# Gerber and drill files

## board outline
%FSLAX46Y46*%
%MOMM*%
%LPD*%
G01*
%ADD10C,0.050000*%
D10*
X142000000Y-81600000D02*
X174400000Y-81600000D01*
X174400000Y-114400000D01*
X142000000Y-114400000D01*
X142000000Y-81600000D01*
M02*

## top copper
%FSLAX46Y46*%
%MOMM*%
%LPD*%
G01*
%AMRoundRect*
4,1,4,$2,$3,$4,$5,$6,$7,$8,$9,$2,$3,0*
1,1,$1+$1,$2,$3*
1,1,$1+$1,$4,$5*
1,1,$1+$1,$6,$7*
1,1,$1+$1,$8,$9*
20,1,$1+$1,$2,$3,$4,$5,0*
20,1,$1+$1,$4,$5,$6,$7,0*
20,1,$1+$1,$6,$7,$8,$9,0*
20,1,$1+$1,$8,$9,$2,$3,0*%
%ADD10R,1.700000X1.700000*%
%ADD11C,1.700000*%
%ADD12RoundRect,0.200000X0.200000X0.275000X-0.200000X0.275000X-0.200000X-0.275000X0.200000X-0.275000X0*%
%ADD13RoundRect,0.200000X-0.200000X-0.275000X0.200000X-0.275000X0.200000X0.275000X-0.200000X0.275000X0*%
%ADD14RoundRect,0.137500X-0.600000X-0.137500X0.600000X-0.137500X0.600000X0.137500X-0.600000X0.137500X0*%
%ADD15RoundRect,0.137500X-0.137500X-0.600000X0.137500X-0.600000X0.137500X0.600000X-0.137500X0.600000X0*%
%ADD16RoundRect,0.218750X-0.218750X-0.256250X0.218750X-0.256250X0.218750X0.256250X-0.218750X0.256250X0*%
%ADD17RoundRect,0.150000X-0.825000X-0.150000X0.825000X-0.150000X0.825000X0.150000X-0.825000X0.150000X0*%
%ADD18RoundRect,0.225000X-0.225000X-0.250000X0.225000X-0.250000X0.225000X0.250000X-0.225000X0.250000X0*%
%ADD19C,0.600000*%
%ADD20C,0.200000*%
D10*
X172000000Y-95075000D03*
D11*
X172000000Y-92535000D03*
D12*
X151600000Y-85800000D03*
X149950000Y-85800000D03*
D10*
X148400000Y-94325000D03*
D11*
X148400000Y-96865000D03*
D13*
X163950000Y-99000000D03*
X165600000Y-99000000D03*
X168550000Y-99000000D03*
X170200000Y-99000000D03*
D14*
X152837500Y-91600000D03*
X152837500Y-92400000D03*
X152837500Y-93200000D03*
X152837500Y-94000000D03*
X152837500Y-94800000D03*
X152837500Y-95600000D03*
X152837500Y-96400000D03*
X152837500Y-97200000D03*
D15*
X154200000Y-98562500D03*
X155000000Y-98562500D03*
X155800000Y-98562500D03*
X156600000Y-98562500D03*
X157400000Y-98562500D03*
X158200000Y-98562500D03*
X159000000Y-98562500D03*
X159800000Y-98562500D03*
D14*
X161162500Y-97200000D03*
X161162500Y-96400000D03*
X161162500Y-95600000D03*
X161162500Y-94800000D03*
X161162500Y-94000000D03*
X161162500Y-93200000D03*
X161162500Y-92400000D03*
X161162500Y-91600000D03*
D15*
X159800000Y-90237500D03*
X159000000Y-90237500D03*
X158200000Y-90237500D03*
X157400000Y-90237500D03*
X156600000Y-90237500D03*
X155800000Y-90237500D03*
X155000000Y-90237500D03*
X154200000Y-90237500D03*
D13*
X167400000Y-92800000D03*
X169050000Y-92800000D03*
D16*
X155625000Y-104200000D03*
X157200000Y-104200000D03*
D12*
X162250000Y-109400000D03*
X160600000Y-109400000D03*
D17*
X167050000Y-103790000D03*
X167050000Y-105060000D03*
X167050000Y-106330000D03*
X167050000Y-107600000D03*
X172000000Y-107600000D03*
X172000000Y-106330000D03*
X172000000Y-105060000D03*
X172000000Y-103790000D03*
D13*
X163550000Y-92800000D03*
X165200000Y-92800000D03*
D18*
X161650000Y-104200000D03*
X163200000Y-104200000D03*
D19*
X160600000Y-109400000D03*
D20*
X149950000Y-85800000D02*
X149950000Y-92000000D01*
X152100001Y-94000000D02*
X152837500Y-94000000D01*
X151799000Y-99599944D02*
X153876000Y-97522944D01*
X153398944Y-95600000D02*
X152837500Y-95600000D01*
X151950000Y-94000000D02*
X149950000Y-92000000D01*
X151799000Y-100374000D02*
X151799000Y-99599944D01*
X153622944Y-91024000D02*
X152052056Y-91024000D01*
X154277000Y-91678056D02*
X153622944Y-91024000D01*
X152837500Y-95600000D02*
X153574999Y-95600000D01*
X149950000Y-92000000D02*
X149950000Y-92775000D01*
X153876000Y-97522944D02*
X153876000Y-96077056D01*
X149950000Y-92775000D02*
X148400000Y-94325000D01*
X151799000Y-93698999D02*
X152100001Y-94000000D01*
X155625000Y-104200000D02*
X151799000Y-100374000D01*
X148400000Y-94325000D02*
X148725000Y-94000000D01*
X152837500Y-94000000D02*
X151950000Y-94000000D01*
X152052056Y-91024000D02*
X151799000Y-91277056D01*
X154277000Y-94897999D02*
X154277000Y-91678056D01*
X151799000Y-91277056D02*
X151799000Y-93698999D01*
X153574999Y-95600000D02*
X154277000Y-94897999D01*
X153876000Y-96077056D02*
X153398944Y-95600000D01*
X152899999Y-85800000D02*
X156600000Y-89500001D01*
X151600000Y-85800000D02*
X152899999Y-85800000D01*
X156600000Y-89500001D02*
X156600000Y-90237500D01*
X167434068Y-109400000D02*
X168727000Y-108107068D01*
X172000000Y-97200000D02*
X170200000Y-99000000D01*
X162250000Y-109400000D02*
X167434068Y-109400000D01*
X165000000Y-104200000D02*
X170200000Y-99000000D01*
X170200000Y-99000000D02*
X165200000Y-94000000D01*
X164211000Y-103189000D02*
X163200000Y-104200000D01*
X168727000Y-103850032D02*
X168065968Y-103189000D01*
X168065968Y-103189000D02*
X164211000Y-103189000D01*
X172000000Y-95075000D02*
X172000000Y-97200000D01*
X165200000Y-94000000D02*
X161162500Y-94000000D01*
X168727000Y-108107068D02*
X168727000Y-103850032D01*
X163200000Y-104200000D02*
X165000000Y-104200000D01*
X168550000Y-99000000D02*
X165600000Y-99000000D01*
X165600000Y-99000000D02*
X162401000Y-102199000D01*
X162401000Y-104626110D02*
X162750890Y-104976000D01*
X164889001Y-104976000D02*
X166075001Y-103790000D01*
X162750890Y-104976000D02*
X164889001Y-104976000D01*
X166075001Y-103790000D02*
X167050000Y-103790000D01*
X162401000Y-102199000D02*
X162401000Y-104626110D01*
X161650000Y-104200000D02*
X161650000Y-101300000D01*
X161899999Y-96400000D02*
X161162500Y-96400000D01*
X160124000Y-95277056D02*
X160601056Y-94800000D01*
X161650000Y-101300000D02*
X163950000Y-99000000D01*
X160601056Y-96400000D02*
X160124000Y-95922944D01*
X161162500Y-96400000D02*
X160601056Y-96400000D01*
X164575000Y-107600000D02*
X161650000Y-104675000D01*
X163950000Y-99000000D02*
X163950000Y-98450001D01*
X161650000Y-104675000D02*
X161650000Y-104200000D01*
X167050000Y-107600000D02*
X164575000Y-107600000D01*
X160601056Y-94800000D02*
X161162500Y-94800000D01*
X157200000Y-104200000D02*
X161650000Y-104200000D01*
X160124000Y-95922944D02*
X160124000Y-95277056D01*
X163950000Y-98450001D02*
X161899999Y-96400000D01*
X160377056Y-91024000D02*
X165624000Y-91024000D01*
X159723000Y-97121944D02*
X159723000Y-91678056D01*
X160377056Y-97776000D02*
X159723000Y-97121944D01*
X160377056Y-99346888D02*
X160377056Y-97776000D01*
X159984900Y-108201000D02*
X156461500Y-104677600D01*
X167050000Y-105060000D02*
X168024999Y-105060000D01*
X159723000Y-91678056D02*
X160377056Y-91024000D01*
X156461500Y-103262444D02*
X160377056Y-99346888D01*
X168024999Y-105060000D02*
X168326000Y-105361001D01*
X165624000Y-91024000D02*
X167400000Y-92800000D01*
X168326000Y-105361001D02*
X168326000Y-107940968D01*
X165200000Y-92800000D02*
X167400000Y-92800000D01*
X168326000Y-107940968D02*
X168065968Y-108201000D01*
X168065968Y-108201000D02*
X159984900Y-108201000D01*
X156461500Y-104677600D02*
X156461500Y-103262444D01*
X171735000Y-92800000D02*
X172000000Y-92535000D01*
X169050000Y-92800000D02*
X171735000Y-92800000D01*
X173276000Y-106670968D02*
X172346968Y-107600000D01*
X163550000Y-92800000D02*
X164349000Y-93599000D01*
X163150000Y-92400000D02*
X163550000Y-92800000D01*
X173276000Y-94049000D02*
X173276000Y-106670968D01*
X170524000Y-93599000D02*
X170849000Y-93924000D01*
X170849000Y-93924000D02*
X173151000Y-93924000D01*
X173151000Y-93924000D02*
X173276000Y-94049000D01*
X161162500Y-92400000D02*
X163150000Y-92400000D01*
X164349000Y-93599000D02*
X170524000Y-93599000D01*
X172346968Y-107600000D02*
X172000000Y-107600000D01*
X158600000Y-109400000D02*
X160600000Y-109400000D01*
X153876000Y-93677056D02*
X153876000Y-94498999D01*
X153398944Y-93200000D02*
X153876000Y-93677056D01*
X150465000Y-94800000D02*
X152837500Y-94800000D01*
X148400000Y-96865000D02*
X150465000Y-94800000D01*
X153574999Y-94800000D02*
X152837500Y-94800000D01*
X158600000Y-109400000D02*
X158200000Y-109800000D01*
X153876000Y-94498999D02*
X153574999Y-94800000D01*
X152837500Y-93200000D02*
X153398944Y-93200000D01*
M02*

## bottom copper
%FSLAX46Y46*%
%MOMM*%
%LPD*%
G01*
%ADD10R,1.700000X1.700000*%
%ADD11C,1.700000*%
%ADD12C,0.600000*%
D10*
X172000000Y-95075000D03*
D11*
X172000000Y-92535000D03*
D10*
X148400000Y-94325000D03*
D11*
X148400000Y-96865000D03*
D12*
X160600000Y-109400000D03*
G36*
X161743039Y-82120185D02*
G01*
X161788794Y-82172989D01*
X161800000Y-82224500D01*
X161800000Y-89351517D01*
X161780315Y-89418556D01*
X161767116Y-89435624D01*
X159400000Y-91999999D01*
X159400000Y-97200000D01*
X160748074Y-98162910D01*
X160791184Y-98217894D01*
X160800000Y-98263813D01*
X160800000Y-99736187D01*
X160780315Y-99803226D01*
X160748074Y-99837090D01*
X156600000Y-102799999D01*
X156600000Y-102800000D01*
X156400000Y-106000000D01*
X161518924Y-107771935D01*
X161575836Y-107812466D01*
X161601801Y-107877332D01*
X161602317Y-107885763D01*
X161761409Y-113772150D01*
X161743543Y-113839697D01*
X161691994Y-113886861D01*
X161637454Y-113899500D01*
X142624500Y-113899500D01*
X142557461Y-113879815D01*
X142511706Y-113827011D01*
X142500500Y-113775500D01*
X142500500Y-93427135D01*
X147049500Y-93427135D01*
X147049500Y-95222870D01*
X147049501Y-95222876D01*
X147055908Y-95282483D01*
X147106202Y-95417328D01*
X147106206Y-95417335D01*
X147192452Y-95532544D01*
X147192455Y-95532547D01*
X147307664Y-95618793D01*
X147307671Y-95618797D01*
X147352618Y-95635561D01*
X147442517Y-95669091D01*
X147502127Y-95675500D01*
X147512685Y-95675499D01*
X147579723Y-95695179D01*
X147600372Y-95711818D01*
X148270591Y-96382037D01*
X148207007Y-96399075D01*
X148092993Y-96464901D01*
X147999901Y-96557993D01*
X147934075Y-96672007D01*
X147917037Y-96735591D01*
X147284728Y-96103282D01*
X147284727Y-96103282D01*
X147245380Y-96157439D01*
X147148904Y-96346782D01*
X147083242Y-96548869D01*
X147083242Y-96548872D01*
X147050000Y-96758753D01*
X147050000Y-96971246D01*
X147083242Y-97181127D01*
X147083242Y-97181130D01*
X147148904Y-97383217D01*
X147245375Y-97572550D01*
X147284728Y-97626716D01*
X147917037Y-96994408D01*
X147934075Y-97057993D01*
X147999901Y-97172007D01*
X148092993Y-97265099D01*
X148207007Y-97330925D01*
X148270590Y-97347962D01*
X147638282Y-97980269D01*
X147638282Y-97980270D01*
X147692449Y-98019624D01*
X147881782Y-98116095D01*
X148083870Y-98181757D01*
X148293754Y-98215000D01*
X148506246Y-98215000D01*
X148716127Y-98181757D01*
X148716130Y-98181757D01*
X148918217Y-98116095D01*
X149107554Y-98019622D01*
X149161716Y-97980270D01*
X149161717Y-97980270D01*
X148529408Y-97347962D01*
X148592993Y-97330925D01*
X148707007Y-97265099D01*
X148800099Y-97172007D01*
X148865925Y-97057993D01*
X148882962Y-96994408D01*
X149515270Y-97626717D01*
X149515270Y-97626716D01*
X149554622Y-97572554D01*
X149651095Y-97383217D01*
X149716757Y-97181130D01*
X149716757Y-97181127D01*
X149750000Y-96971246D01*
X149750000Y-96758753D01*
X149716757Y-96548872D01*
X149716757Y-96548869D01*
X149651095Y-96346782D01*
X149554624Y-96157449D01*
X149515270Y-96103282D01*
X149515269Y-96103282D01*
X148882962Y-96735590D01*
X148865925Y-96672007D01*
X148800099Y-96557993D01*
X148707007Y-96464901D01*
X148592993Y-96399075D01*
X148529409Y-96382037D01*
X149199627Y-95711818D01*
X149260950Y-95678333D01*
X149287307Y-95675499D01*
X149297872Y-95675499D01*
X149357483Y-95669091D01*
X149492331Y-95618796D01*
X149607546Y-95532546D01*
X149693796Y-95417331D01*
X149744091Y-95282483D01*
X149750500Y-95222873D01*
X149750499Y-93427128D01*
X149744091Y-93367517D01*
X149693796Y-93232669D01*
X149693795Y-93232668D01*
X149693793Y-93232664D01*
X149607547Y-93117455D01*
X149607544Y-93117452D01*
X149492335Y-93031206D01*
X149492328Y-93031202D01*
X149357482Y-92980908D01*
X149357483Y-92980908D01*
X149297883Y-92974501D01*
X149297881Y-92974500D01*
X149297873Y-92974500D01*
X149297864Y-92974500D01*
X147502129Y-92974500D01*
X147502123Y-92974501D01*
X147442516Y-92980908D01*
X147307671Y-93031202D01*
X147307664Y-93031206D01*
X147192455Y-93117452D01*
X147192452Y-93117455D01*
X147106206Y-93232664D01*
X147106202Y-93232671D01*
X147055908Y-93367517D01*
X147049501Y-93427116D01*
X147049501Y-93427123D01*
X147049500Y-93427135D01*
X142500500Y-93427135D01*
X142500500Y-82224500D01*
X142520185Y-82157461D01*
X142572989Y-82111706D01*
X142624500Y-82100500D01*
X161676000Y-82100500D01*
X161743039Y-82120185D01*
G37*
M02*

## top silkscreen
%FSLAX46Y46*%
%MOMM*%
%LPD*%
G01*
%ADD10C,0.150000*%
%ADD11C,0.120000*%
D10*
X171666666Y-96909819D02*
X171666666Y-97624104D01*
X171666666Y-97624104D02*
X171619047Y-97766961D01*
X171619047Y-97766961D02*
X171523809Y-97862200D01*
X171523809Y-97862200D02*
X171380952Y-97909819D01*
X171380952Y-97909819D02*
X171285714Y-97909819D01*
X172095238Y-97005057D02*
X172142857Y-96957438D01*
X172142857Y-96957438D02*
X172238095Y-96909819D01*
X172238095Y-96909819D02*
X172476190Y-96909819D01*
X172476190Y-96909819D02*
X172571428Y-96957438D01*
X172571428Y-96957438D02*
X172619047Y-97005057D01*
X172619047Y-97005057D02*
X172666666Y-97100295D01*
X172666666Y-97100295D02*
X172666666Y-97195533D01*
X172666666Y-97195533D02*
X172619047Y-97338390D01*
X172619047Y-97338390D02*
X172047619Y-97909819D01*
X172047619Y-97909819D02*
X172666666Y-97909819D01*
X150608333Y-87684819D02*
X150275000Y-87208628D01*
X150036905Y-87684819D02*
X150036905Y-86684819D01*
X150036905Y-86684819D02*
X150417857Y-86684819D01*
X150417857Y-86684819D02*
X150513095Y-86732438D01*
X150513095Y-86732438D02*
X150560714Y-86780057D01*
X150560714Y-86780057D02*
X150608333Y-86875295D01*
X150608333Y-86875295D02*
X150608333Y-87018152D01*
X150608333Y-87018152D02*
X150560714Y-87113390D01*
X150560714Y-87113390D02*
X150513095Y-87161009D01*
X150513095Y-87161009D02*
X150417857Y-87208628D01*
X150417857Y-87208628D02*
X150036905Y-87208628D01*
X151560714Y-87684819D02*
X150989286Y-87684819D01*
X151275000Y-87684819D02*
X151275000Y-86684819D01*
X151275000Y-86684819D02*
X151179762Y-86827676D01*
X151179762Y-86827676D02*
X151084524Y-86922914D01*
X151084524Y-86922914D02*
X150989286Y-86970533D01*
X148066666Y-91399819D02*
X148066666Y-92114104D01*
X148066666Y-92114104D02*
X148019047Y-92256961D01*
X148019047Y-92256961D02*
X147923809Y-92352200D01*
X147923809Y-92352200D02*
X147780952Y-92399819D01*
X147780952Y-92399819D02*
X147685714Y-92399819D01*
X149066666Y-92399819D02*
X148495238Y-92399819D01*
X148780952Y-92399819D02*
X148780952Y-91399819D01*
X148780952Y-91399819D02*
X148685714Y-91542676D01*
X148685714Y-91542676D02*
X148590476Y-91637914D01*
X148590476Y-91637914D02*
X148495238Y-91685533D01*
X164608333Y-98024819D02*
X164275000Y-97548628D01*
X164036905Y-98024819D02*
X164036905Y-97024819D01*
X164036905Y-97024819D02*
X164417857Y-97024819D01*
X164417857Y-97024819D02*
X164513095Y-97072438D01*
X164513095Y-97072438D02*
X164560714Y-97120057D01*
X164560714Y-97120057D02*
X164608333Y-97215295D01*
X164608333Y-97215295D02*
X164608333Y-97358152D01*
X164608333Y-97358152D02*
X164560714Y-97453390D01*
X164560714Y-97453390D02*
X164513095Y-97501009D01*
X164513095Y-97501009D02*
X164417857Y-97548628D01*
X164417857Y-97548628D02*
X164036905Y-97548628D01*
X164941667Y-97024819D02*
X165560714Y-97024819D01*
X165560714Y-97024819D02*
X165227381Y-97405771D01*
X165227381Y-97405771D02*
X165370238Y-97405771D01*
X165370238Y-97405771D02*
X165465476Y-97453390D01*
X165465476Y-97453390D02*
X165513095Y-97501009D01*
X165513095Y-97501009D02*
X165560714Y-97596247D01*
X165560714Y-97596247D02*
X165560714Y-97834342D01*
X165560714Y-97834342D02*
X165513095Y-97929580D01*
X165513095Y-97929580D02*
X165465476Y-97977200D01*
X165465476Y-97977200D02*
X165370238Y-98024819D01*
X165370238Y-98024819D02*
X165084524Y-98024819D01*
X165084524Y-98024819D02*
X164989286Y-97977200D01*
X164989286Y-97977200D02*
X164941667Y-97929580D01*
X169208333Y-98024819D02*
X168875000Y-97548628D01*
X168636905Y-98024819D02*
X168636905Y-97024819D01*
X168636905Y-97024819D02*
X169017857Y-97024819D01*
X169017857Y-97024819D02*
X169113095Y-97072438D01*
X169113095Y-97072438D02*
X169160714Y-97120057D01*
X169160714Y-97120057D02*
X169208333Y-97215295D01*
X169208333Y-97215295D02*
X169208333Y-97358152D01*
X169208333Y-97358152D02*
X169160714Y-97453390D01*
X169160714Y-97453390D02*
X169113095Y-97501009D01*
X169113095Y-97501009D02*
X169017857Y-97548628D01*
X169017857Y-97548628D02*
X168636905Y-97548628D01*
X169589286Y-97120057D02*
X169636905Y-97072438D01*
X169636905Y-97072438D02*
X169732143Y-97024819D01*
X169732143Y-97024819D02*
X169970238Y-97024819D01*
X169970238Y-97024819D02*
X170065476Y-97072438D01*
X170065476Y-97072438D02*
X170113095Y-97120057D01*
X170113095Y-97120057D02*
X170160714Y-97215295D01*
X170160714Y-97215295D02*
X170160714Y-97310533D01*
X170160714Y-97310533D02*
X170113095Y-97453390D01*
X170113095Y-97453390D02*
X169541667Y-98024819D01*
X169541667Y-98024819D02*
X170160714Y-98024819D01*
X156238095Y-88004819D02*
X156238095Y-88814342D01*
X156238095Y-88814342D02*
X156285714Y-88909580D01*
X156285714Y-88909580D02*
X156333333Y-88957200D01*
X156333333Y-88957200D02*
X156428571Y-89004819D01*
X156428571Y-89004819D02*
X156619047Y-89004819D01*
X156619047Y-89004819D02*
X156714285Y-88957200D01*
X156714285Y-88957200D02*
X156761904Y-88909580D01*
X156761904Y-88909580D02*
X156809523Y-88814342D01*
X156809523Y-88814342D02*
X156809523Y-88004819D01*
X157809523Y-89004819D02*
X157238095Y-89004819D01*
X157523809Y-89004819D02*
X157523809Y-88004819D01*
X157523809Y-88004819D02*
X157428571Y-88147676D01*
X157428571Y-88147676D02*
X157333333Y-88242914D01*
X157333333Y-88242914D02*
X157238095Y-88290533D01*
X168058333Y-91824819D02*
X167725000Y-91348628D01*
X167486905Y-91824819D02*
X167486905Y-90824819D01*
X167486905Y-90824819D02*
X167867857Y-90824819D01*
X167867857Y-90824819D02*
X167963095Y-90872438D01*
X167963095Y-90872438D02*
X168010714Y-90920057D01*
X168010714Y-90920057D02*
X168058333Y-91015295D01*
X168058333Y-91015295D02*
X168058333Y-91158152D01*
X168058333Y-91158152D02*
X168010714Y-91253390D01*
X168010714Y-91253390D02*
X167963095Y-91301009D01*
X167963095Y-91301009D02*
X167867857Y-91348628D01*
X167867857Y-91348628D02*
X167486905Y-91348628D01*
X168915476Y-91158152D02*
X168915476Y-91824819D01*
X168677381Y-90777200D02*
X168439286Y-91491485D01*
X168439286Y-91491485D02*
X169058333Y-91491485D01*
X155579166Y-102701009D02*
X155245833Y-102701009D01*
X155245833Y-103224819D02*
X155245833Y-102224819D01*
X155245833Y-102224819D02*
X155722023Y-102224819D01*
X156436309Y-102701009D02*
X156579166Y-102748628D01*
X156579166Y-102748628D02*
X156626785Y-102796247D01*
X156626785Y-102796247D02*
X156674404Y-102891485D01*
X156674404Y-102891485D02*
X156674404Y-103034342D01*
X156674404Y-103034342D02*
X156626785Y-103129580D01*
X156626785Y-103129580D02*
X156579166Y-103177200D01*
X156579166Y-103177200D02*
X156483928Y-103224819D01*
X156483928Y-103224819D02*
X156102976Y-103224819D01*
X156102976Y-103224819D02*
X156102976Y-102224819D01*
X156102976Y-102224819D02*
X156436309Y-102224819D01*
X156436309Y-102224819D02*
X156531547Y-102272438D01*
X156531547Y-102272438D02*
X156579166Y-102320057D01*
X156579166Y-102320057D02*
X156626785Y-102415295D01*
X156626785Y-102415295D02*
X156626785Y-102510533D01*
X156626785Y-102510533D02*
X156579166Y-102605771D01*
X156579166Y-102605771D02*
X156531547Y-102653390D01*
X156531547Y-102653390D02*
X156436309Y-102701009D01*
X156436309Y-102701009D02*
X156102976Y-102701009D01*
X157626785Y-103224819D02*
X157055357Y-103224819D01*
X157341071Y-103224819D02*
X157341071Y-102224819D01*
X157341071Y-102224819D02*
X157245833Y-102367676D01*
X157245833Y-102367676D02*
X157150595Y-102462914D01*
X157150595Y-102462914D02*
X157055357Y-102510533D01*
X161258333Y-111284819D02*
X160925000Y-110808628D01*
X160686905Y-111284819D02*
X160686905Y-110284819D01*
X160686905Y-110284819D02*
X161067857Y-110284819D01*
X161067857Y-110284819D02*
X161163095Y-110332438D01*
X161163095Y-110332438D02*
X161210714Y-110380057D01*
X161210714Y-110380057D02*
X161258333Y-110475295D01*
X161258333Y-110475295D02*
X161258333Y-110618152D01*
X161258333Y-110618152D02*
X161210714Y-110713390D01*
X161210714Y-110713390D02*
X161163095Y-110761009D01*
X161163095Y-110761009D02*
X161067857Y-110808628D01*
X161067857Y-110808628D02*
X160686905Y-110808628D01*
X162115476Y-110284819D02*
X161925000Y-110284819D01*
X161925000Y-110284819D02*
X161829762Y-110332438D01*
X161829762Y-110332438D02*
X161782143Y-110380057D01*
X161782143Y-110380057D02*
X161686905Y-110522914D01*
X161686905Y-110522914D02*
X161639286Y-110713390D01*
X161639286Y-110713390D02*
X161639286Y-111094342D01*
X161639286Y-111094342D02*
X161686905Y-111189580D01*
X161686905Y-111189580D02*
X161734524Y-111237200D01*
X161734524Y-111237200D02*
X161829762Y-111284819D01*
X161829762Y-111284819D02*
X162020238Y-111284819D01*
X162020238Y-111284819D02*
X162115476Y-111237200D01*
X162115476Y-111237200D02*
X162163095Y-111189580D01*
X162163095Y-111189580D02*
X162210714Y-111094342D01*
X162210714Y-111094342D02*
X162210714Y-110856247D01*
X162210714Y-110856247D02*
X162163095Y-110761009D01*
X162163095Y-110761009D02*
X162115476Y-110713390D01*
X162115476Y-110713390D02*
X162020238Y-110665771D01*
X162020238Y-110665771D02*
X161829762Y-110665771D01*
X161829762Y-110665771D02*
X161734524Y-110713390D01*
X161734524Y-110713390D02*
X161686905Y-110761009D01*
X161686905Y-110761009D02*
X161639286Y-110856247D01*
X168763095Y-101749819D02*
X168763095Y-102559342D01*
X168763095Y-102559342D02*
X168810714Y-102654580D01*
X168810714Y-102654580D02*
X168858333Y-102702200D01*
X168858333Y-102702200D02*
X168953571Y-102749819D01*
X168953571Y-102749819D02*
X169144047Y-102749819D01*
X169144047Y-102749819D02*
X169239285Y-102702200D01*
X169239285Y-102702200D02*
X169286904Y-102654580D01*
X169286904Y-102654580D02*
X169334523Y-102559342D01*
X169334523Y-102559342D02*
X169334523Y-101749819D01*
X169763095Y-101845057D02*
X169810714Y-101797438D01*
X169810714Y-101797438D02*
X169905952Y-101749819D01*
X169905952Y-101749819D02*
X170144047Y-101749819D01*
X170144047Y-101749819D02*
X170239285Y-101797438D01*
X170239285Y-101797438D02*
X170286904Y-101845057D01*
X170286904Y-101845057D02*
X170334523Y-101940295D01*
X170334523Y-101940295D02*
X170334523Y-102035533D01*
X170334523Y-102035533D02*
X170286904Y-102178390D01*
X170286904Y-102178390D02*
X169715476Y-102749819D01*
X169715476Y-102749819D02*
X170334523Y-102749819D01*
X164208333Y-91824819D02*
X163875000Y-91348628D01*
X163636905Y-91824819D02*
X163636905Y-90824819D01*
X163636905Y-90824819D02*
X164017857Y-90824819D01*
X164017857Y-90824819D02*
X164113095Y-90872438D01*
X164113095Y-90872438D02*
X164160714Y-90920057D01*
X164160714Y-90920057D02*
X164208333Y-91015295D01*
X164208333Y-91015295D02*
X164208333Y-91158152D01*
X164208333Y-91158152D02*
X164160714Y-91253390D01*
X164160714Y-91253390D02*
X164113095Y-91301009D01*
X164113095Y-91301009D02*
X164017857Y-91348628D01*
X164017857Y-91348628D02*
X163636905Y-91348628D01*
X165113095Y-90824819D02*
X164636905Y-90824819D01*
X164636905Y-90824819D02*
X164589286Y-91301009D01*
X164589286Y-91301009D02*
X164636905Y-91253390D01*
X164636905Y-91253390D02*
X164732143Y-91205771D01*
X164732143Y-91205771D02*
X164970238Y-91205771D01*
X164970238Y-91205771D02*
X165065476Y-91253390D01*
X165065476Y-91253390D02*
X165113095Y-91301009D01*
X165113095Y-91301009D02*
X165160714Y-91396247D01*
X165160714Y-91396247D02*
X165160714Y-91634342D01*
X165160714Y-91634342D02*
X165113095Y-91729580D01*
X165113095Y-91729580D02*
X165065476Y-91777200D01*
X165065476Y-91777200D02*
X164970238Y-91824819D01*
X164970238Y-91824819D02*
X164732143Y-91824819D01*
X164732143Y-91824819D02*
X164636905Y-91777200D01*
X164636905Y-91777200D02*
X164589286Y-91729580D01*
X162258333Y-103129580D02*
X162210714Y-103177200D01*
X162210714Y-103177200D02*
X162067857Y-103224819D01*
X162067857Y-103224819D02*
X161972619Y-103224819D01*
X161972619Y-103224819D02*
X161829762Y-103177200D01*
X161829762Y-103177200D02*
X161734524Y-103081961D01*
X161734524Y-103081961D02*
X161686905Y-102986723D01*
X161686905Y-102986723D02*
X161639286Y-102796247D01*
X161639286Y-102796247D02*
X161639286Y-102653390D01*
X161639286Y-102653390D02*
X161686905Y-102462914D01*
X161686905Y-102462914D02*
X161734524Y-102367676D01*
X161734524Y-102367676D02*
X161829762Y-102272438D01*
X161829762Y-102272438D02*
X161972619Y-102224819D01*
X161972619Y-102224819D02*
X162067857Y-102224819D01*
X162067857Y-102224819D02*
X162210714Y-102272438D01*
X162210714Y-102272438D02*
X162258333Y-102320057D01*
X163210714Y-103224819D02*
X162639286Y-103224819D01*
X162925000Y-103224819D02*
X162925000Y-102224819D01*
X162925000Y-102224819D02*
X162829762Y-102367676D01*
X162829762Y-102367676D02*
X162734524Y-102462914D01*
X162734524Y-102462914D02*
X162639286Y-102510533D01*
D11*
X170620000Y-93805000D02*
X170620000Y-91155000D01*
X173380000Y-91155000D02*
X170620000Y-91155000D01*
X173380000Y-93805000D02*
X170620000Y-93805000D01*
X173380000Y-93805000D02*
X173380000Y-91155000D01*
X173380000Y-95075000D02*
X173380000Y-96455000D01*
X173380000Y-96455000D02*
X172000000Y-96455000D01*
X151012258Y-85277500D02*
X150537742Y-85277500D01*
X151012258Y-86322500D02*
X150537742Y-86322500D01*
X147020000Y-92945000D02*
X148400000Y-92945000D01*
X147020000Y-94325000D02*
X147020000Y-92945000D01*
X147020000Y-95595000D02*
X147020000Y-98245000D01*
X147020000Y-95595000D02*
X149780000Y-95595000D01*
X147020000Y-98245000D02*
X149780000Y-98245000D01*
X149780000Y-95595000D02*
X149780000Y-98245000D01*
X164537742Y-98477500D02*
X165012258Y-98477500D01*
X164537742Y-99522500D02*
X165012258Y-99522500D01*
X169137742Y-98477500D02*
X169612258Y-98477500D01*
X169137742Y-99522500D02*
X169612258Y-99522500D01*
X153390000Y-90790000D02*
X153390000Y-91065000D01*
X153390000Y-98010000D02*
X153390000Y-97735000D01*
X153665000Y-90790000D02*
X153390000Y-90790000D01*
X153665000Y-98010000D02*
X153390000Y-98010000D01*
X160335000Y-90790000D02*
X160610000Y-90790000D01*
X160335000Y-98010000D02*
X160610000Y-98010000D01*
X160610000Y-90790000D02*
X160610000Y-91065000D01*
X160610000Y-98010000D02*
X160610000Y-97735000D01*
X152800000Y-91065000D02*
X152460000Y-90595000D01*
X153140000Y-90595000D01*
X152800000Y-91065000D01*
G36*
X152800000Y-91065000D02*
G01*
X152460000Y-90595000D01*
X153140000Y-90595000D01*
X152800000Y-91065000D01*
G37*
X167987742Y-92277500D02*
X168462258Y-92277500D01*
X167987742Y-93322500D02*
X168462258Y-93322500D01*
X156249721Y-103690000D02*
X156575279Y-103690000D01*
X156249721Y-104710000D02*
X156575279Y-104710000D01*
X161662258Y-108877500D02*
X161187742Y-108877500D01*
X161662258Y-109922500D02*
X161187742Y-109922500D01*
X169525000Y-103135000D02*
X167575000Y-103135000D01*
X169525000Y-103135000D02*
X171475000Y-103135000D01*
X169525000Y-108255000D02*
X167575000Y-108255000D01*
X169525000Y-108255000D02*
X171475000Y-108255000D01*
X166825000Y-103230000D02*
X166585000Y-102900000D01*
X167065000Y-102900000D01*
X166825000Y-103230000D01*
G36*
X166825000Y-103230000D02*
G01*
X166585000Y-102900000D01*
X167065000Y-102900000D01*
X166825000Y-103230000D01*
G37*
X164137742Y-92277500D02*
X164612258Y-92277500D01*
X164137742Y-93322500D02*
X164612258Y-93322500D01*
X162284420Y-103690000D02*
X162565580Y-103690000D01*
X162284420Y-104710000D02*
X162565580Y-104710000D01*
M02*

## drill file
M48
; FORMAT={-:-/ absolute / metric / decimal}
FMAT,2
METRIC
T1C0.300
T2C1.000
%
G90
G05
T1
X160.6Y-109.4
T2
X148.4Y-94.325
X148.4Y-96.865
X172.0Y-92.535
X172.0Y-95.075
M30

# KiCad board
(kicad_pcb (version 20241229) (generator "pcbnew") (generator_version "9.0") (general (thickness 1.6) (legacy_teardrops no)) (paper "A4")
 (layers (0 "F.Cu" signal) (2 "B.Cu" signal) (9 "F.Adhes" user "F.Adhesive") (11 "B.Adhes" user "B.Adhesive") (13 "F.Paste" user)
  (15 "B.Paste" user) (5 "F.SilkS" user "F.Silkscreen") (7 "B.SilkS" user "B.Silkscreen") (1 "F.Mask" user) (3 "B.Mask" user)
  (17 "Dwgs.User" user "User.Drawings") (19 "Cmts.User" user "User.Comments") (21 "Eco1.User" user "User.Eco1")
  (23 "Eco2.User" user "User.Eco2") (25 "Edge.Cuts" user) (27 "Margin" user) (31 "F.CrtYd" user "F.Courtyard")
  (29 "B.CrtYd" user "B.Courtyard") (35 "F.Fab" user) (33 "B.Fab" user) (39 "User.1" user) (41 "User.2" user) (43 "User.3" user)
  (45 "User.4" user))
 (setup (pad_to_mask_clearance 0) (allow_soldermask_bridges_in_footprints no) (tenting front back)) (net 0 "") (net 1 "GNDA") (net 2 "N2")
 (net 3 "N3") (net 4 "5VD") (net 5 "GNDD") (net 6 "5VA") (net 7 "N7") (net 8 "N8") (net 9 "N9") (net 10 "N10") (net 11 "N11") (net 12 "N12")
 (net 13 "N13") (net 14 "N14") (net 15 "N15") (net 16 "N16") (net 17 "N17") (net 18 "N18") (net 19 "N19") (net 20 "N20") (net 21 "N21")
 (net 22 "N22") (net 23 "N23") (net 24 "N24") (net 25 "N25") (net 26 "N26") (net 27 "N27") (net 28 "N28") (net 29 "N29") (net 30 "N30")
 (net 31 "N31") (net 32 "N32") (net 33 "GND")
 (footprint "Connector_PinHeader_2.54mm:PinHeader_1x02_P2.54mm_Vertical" (layer "F.Cu") (at 172 95.075 180)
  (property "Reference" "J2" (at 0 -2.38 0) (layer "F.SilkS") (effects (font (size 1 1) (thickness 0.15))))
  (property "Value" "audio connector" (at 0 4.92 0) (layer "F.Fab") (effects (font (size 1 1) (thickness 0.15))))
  (fp_line (start 1.38 1.27) (end 1.38 3.92) (stroke (width 0.12) (type solid)) (layer "F.SilkS"))
  (fp_line (start -1.38 3.92) (end 1.38 3.92) (stroke (width 0.12) (type solid)) (layer "F.SilkS"))
  (fp_line (start -1.38 1.27) (end 1.38 1.27) (stroke (width 0.12) (type solid)) (layer "F.SilkS"))
  (fp_line (start -1.38 1.27) (end -1.38 3.92) (stroke (width 0.12) (type solid)) (layer "F.SilkS"))
  (fp_line (start -1.38 0) (end -1.38 -1.38) (stroke (width 0.12) (type solid)) (layer "F.SilkS"))
  (fp_line (start -1.38 -1.38) (end 0 -1.38) (stroke (width 0.12) (type solid)) (layer "F.SilkS"))
  (pad "1" thru_hole rect (at 0 0 180) (size 1.7 1.7) (drill 1) (layers "*.Cu" "*.Mask") (remove_unused_layers no) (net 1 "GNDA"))
  (pad "2" thru_hole circle (at 0 2.54 180) (size 1.7 1.7) (drill 1) (layers "*.Cu" "*.Mask") (remove_unused_layers no) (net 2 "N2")))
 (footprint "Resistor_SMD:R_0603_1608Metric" (layer "F.Cu") (at 150.775 85.8 180)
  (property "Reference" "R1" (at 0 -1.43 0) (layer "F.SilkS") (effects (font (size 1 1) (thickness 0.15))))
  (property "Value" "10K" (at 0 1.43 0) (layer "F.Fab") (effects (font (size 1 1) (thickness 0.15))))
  (fp_line (start -0.237258 0.5225) (end 0.237258 0.5225) (stroke (width 0.12) (type solid)) (layer "F.SilkS"))
  (fp_line (start -0.237258 -0.5225) (end 0.237258 -0.5225) (stroke (width 0.12) (type solid)) (layer "F.SilkS"))
  (pad "1" smd roundrect (at -0.825 0 180) (size 0.8 0.95) (layers "F.Cu" "F.Mask" "F.Paste") (roundrect_rratio 0.25) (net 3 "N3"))
  (pad "2" smd roundrect (at 0.825 0 180) (size 0.8 0.95) (layers "F.Cu" "F.Mask" "F.Paste") (roundrect_rratio 0.25) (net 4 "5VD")))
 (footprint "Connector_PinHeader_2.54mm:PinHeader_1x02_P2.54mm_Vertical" (layer "F.Cu") (at 148.4 94.325)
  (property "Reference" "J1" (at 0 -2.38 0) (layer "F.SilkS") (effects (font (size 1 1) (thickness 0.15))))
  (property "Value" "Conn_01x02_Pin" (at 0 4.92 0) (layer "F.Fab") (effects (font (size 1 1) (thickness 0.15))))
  (fp_line (start -1.38 -1.38) (end 0 -1.38) (stroke (width 0.12) (type solid)) (layer "F.SilkS"))
  (fp_line (start -1.38 0) (end -1.38 -1.38) (stroke (width 0.12) (type solid)) (layer "F.SilkS"))
  (fp_line (start -1.38 1.27) (end -1.38 3.92) (stroke (width 0.12) (type solid)) (layer "F.SilkS"))
  (fp_line (start -1.38 1.27) (end 1.38 1.27) (stroke (width 0.12) (type solid)) (layer "F.SilkS"))
  (fp_line (start -1.38 3.92) (end 1.38 3.92) (stroke (width 0.12) (type solid)) (layer "F.SilkS"))
  (fp_line (start 1.38 1.27) (end 1.38 3.92) (stroke (width 0.12) (type solid)) (layer "F.SilkS"))
  (pad "1" thru_hole rect (at 0 0) (size 1.7 1.7) (drill 1) (layers "*.Cu" "*.Mask") (remove_unused_layers no) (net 4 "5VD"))
  (pad "2" thru_hole circle (at 0 2.54) (size 1.7 1.7) (drill 1) (layers "*.Cu" "*.Mask") (remove_unused_layers no) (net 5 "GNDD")))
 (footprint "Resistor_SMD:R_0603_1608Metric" (layer "F.Cu") (at 164.775 99)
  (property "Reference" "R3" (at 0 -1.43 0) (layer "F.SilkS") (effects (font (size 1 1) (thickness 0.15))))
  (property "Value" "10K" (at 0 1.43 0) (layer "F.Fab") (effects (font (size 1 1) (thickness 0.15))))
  (fp_line (start -0.237258 -0.5225) (end 0.237258 -0.5225) (stroke (width 0.12) (type solid)) (layer "F.SilkS"))
  (fp_line (start -0.237258 0.5225) (end 0.237258 0.5225) (stroke (width 0.12) (type solid)) (layer "F.SilkS"))
  (pad "1" smd roundrect (at -0.825 0) (size 0.8 0.95) (layers "F.Cu" "F.Mask" "F.Paste") (roundrect_rratio 0.25) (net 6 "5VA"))
  (pad "2" smd roundrect (at 0.825 0) (size 0.8 0.95) (layers "F.Cu" "F.Mask" "F.Paste") (roundrect_rratio 0.25) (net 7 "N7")))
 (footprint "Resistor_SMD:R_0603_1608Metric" (layer "F.Cu") (at 169.375 99)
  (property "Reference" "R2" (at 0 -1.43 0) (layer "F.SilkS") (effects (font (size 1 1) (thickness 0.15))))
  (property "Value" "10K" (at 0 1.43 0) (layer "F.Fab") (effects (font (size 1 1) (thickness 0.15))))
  (fp_line (start -0.237258 -0.5225) (end 0.237258 -0.5225) (stroke (width 0.12) (type solid)) (layer "F.SilkS"))
  (fp_line (start -0.237258 0.5225) (end 0.237258 0.5225) (stroke (width 0.12) (type solid)) (layer "F.SilkS"))
  (pad "1" smd roundrect (at -0.825 0) (size 0.8 0.95) (layers "F.Cu" "F.Mask" "F.Paste") (roundrect_rratio 0.25) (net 7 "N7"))
  (pad "2" smd roundrect (at 0.825 0) (size 0.8 0.95) (layers "F.Cu" "F.Mask" "F.Paste") (roundrect_rratio 0.25) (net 1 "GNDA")))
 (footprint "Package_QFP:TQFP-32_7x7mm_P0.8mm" (layer "F.Cu") (at 157 94.4)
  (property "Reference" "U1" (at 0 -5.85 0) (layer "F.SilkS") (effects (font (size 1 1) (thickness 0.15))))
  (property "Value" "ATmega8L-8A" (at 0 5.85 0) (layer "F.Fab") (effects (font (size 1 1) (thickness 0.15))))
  (fp_line (start -3.61 -3.61) (end -3.61 -3.335) (stroke (width 0.12) (type solid)) (layer "F.SilkS"))
  (fp_line (start -3.61 3.61) (end -3.61 3.335) (stroke (width 0.12) (type solid)) (layer "F.SilkS"))
  (fp_line (start -3.335 -3.61) (end -3.61 -3.61) (stroke (width 0.12) (type solid)) (layer "F.SilkS"))
  (fp_line (start -3.335 3.61) (end -3.61 3.61) (stroke (width 0.12) (type solid)) (layer "F.SilkS"))
  (fp_line (start 3.335 -3.61) (end 3.61 -3.61) (stroke (width 0.12) (type solid)) (layer "F.SilkS"))
  (fp_line (start 3.335 3.61) (end 3.61 3.61) (stroke (width 0.12) (type solid)) (layer "F.SilkS"))
  (fp_line (start 3.61 -3.61) (end 3.61 -3.335) (stroke (width 0.12) (type solid)) (layer "F.SilkS"))
  (fp_line (start 3.61 3.61) (end 3.61 3.335) (stroke (width 0.12) (type solid)) (layer "F.SilkS"))
  (fp_poly (pts (xy -4.2 -3.335) (xy -4.54 -3.805) (xy -3.86 -3.805)) (stroke (width 0.12) (type solid)) (fill yes) (layer "F.SilkS"))
  (pad "1" smd roundrect (at -4.1625 -2.8) (size 1.475 0.55) (layers "F.Cu" "F.Mask" "F.Paste") (roundrect_rratio 0.25) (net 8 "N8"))
  (pad "2" smd roundrect (at -4.1625 -2) (size 1.475 0.55) (layers "F.Cu" "F.Mask" "F.Paste") (roundrect_rratio 0.25) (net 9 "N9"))
  (pad "3" smd roundrect (at -4.1625 -1.2) (size 1.475 0.55) (layers "F.Cu" "F.Mask" "F.Paste") (roundrect_rratio 0.25) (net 5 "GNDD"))
  (pad "4" smd roundrect (at -4.1625 -0.4) (size 1.475 0.55) (layers "F.Cu" "F.Mask" "F.Paste") (roundrect_rratio 0.25) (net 4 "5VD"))
  (pad "5" smd roundrect (at -4.1625 0.4) (size 1.475 0.55) (layers "F.Cu" "F.Mask" "F.Paste") (roundrect_rratio 0.25) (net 5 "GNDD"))
  (pad "6" smd roundrect (at -4.1625 1.2) (size 1.475 0.55) (layers "F.Cu" "F.Mask" "F.Paste") (roundrect_rratio 0.25) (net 4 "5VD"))
  (pad "7" smd roundrect (at -4.1625 2) (size 1.475 0.55) (layers "F.Cu" "F.Mask" "F.Paste") (roundrect_rratio 0.25) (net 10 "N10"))
  (pad "8" smd roundrect (at -4.1625 2.8) (size 1.475 0.55) (layers "F.Cu" "F.Mask" "F.Paste") (roundrect_rratio 0.25) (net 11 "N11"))
  (pad "9" smd roundrect (at -2.8 4.1625) (size 0.55 1.475) (layers "F.Cu" "F.Mask" "F.Paste") (roundrect_rratio 0.25) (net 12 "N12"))
  (pad "10" smd roundrect (at -2 4.1625) (size 0.55 1.475) (layers "F.Cu" "F.Mask" "F.Paste") (roundrect_rratio 0.25) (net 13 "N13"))
  (pad "11" smd roundrect (at -1.2 4.1625) (size 0.55 1.475) (layers "F.Cu" "F.Mask" "F.Paste") (roundrect_rratio 0.25) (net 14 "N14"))
  (pad "12" smd roundrect (at -0.4 4.1625) (size 0.55 1.475) (layers "F.Cu" "F.Mask" "F.Paste") (roundrect_rratio 0.25) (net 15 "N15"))
  (pad "13" smd roundrect (at 0.4 4.1625) (size 0.55 1.475) (layers "F.Cu" "F.Mask" "F.Paste") (roundrect_rratio 0.25) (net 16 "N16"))
  (pad "14" smd roundrect (at 1.2 4.1625) (size 0.55 1.475) (layers "F.Cu" "F.Mask" "F.Paste") (roundrect_rratio 0.25) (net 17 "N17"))
  (pad "15" smd roundrect (at 2 4.1625) (size 0.55 1.475) (layers "F.Cu" "F.Mask" "F.Paste") (roundrect_rratio 0.25) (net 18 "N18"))
  (pad "16" smd roundrect (at 2.8 4.1625) (size 0.55 1.475) (layers "F.Cu" "F.Mask" "F.Paste") (roundrect_rratio 0.25) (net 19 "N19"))
  (pad "17" smd roundrect (at 4.1625 2.8) (size 1.475 0.55) (layers "F.Cu" "F.Mask" "F.Paste") (roundrect_rratio 0.25) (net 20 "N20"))
  (pad "18" smd roundrect (at 4.1625 2) (size 1.475 0.55) (layers "F.Cu" "F.Mask" "F.Paste") (roundrect_rratio 0.25) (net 6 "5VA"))
  (pad "19" smd roundrect (at 4.1625 1.2) (size 1.475 0.55) (layers "F.Cu" "F.Mask" "F.Paste") (roundrect_rratio 0.25) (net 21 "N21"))
  (pad "20" smd roundrect (at 4.1625 0.4) (size 1.475 0.55) (layers "F.Cu" "F.Mask" "F.Paste") (roundrect_rratio 0.25) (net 6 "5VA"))
  (pad "21" smd roundrect (at 4.1625 -0.4) (size 1.475 0.55) (layers "F.Cu" "F.Mask" "F.Paste") (roundrect_rratio 0.25) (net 1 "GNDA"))
  (pad "22" smd roundrect (at 4.1625 -1.2) (size 1.475 0.55) (layers "F.Cu" "F.Mask" "F.Paste") (roundrect_rratio 0.25) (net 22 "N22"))
  (pad "23" smd roundrect (at 4.1625 -2) (size 1.475 0.55) (layers "F.Cu" "F.Mask" "F.Paste") (roundrect_rratio 0.25) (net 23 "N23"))
  (pad "24" smd roundrect (at 4.1625 -2.8) (size 1.475 0.55) (layers "F.Cu" "F.Mask" "F.Paste") (roundrect_rratio 0.25) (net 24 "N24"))
  (pad "25" smd roundrect (at 2.8 -4.1625) (size 0.55 1.475) (layers "F.Cu" "F.Mask" "F.Paste") (roundrect_rratio 0.25) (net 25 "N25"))
  (pad "26" smd roundrect (at 2 -4.1625) (size 0.55 1.475) (layers "F.Cu" "F.Mask" "F.Paste") (roundrect_rratio 0.25) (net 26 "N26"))
  (pad "27" smd roundrect (at 1.2 -4.1625) (size 0.55 1.475) (layers "F.Cu" "F.Mask" "F.Paste") (roundrect_rratio 0.25) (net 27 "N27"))
  (pad "28" smd roundrect (at 0.4 -4.1625) (size 0.55 1.475) (layers "F.Cu" "F.Mask" "F.Paste") (roundrect_rratio 0.25) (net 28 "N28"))
  (pad "29" smd roundrect (at -0.4 -4.1625) (size 0.55 1.475) (layers "F.Cu" "F.Mask" "F.Paste") (roundrect_rratio 0.25) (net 3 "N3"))
  (pad "30" smd roundrect (at -1.2 -4.1625) (size 0.55 1.475) (layers "F.Cu" "F.Mask" "F.Paste") (roundrect_rratio 0.25) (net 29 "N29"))
  (pad "31" smd roundrect (at -2 -4.1625) (size 0.55 1.475) (layers "F.Cu" "F.Mask" "F.Paste") (roundrect_rratio 0.25) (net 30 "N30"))
  (pad "32" smd roundrect (at -2.8 -4.1625) (size 0.55 1.475) (layers "F.Cu" "F.Mask" "F.Paste") (roundrect_rratio 0.25) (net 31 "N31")))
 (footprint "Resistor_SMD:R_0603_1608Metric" (layer "F.Cu") (at 168.225 92.8)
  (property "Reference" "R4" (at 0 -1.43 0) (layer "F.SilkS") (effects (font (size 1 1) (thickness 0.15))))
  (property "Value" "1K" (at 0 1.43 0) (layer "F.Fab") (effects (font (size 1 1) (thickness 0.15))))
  (fp_line (start -0.237258 -0.5225) (end 0.237258 -0.5225) (stroke (width 0.12) (type solid)) (layer "F.SilkS"))
  (fp_line (start -0.237258 0.5225) (end 0.237258 0.5225) (stroke (width 0.12) (type solid)) (layer "F.SilkS"))
  (pad "1" smd roundrect (at -0.825 0) (size 0.8 0.95) (layers "F.Cu" "F.Mask" "F.Paste") (roundrect_rratio 0.25) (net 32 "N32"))
  (pad "2" smd roundrect (at 0.825 0) (size 0.8 0.95) (layers "F.Cu" "F.Mask" "F.Paste") (roundrect_rratio 0.25) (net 2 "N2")))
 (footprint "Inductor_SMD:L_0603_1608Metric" (layer "F.Cu") (at 156.4125 104.2)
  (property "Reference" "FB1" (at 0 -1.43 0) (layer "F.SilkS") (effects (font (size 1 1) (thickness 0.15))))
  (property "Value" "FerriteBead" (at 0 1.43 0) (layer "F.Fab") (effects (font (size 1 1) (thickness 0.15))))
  (fp_line (start -0.162779 -0.51) (end 0.162779 -0.51) (stroke (width 0.12) (type solid)) (layer "F.SilkS"))
  (fp_line (start -0.162779 0.51) (end 0.162779 0.51) (stroke (width 0.12) (type solid)) (layer "F.SilkS"))
  (pad "1" smd roundrect (at -0.7875 0) (size 0.875 0.95) (layers "F.Cu" "F.Mask" "F.Paste") (roundrect_rratio 0.25) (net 4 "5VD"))
  (pad "2" smd roundrect (at 0.7875 0) (size 0.875 0.95) (layers "F.Cu" "F.Mask" "F.Paste") (roundrect_rratio 0.25) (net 6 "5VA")))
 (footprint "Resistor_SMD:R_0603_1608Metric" (layer "F.Cu") (at 161.425 109.4 180)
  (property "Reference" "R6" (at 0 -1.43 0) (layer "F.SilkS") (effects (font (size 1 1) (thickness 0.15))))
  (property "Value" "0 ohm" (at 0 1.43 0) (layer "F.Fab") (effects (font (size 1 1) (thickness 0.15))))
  (fp_line (start -0.237258 0.5225) (end 0.237258 0.5225) (stroke (width 0.12) (type solid)) (layer "F.SilkS"))
  (fp_line (start -0.237258 -0.5225) (end 0.237258 -0.5225) (stroke (width 0.12) (type solid)) (layer "F.SilkS"))
  (pad "1" smd roundrect (at -0.825 0 180) (size 0.8 0.95) (layers "F.Cu" "F.Mask" "F.Paste") (roundrect_rratio 0.25) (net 1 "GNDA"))
  (pad "2" smd roundrect (at 0.825 0 180) (size 0.8 0.95) (layers "F.Cu" "F.Mask" "F.Paste") (roundrect_rratio 0.25) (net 5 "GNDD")))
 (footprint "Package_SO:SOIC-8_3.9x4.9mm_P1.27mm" (layer "F.Cu") (at 169.525 105.695)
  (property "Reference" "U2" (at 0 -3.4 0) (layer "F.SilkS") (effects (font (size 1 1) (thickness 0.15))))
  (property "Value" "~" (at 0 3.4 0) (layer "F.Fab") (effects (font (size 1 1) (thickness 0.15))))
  (fp_line (start 0 -2.56) (end -1.95 -2.56) (stroke (width 0.12) (type solid)) (layer "F.SilkS"))
  (fp_line (start 0 -2.56) (end 1.95 -2.56) (stroke (width 0.12) (type solid)) (layer "F.SilkS"))
  (fp_line (start 0 2.56) (end -1.95 2.56) (stroke (width 0.12) (type solid)) (layer "F.SilkS"))
  (fp_line (start 0 2.56) (end 1.95 2.56) (stroke (width 0.12) (type solid)) (layer "F.SilkS"))
  (fp_poly (pts (xy -2.7 -2.465) (xy -2.94 -2.795) (xy -2.46 -2.795)) (stroke (width 0.12) (type solid)) (fill yes) (layer "F.SilkS"))
  (pad "1" smd roundrect (at -2.475 -1.905) (size 1.95 0.6) (layers "F.Cu" "F.Mask" "F.Paste") (roundrect_rratio 0.25) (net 7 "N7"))
  (pad "2" smd roundrect (at -2.475 -0.635) (size 1.95 0.6) (layers "F.Cu" "F.Mask" "F.Paste") (roundrect_rratio 0.25) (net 32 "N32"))
  (pad "3" smd roundrect (at -2.475 0.635) (size 1.95 0.6) (layers "F.Cu" "F.Mask" "F.Paste") (roundrect_rratio 0.25) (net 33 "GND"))
  (pad "4" smd roundrect (at -2.475 1.905) (size 1.95 0.6) (layers "F.Cu" "F.Mask" "F.Paste") (roundrect_rratio 0.25) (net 6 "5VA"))
  (pad "5" smd roundrect (at 2.475 1.905) (size 1.95 0.6) (layers "F.Cu" "F.Mask" "F.Paste") (roundrect_rratio 0.25) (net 23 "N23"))
  (pad "6" smd roundrect (at 2.475 0.635) (size 1.95 0.6) (layers "F.Cu" "F.Mask" "F.Paste") (roundrect_rratio 0.25))
  (pad "7" smd roundrect (at 2.475 -0.635) (size 1.95 0.6) (layers "F.Cu" "F.Mask" "F.Paste") (roundrect_rratio 0.25))
  (pad "8" smd roundrect (at 2.475 -1.905) (size 1.95 0.6) (layers "F.Cu" "F.Mask" "F.Paste") (roundrect_rratio 0.25)))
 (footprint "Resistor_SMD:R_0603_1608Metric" (layer "F.Cu") (at 164.375 92.8)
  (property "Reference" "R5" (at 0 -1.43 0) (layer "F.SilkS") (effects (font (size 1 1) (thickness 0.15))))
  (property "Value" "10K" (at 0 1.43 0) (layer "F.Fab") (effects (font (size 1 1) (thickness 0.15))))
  (fp_line (start -0.237258 -0.5225) (end 0.237258 -0.5225) (stroke (width 0.12) (type solid)) (layer "F.SilkS"))
  (fp_line (start -0.237258 0.5225) (end 0.237258 0.5225) (stroke (width 0.12) (type solid)) (layer "F.SilkS"))
  (pad "1" smd roundrect (at -0.825 0) (size 0.8 0.95) (layers "F.Cu" "F.Mask" "F.Paste") (roundrect_rratio 0.25) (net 23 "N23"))
  (pad "2" smd roundrect (at 0.825 0) (size 0.8 0.95) (layers "F.Cu" "F.Mask" "F.Paste") (roundrect_rratio 0.25) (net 32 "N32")))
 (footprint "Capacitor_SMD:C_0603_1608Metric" (layer "F.Cu") (at 162.425 104.2)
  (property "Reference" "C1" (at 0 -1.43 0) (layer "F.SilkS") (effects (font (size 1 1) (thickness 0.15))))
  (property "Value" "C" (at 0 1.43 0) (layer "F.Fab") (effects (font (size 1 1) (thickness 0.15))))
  (fp_line (start -0.14058 -0.51) (end 0.14058 -0.51) (stroke (width 0.12) (type solid)) (layer "F.SilkS"))
  (fp_line (start -0.14058 0.51) (end 0.14058 0.51) (stroke (width 0.12) (type solid)) (layer "F.SilkS"))
  (pad "1" smd roundrect (at -0.775 0) (size 0.9 0.95) (layers "F.Cu" "F.Mask" "F.Paste") (roundrect_rratio 0.25) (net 6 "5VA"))
  (pad "2" smd roundrect (at 0.775 0) (size 0.9 0.95) (layers "F.Cu" "F.Mask" "F.Paste") (roundrect_rratio 0.25) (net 1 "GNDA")))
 (gr_rect (start 142 81.6) (end 174.4 114.4) (stroke (width 0.05) (type default)) (fill no) (layer "Edge.Cuts"))
 (segment (start 149.95 85.8) (end 149.95 92) (width 0.2) (layer "F.Cu") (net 4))
 (segment (start 152.100001 94) (end 152.8375 94) (width 0.2) (layer "F.Cu") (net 4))
 (segment (start 151.799 99.599944) (end 153.876 97.522944) (width 0.2) (layer "F.Cu") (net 4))
 (segment (start 153.398944 95.6) (end 152.8375 95.6) (width 0.2) (layer "F.Cu") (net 4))
 (segment (start 151.95 94) (end 149.95 92) (width 0.2) (layer "F.Cu") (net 4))
 (segment (start 151.799 100.374) (end 151.799 99.599944) (width 0.2) (layer "F.Cu") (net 4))
 (segment (start 153.622944 91.024) (end 152.052056 91.024) (width 0.2) (layer "F.Cu") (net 4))
 (segment (start 154.277 91.678056) (end 153.622944 91.024) (width 0.2) (layer "F.Cu") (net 4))
 (segment (start 152.8375 95.6) (end 153.574999 95.6) (width 0.2) (layer "F.Cu") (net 4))
 (segment (start 149.95 92) (end 149.95 92.775) (width 0.2) (layer "F.Cu") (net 4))
 (segment (start 153.876 97.522944) (end 153.876 96.077056) (width 0.2) (layer "F.Cu") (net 4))
 (segment (start 149.95 92.775) (end 148.4 94.325) (width 0.2) (layer "F.Cu") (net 4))
 (segment (start 151.799 93.698999) (end 152.100001 94) (width 0.2) (layer "F.Cu") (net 4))
 (segment (start 155.625 104.2) (end 151.799 100.374) (width 0.2) (layer "F.Cu") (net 4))
 (segment (start 148.4 94.325) (end 148.725 94) (width 0.2) (layer "F.Cu") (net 4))
 (segment (start 152.8375 94) (end 151.95 94) (width 0.2) (layer "F.Cu") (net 4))
 (segment (start 152.052056 91.024) (end 151.799 91.277056) (width 0.2) (layer "F.Cu") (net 4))
 (segment (start 154.277 94.897999) (end 154.277 91.678056) (width 0.2) (layer "F.Cu") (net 4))
 (segment (start 151.799 91.277056) (end 151.799 93.698999) (width 0.2) (layer "F.Cu") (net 4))
 (segment (start 153.574999 95.6) (end 154.277 94.897999) (width 0.2) (layer "F.Cu") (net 4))
 (segment (start 153.876 96.077056) (end 153.398944 95.6) (width 0.2) (layer "F.Cu") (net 4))
 (segment (start 152.899999 85.8) (end 156.6 89.500001) (width 0.2) (layer "F.Cu") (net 3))
 (segment (start 151.6 85.8) (end 152.899999 85.8) (width 0.2) (layer "F.Cu") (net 3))
 (segment (start 156.6 89.500001) (end 156.6 90.2375) (width 0.2) (layer "F.Cu") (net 3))
 (segment (start 167.434068 109.4) (end 168.727 108.107068) (width 0.2) (layer "F.Cu") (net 1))
 (segment (start 172 97.2) (end 170.2 99) (width 0.2) (layer "F.Cu") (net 1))
 (segment (start 162.25 109.4) (end 167.434068 109.4) (width 0.2) (layer "F.Cu") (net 1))
 (segment (start 165 104.2) (end 170.2 99) (width 0.2) (layer "F.Cu") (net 1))
 (segment (start 170.2 99) (end 165.2 94) (width 0.2) (layer "F.Cu") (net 1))
 (segment (start 164.211 103.189) (end 163.2 104.2) (width 0.2) (layer "F.Cu") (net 1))
 (segment (start 168.727 103.850032) (end 168.065968 103.189) (width 0.2) (layer "F.Cu") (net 1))
 (segment (start 168.065968 103.189) (end 164.211 103.189) (width 0.2) (layer "F.Cu") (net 1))
 (segment (start 172 95.075) (end 172 97.2) (width 0.2) (layer "F.Cu") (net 1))
 (segment (start 165.2 94) (end 161.1625 94) (width 0.2) (layer "F.Cu") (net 1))
 (segment (start 168.727 108.107068) (end 168.727 103.850032) (width 0.2) (layer "F.Cu") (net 1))
 (segment (start 163.2 104.2) (end 165 104.2) (width 0.2) (layer "F.Cu") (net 1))
 (segment (start 168.55 99) (end 165.6 99) (width 0.2) (layer "F.Cu") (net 7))
 (segment (start 165.6 99) (end 162.401 102.199) (width 0.2) (layer "F.Cu") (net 7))
 (segment (start 162.401 104.62611) (end 162.75089 104.976) (width 0.2) (layer "F.Cu") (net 7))
 (segment (start 164.889001 104.976) (end 166.075001 103.79) (width 0.2) (layer "F.Cu") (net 7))
 (segment (start 162.75089 104.976) (end 164.889001 104.976) (width 0.2) (layer "F.Cu") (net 7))
 (segment (start 166.075001 103.79) (end 167.05 103.79) (width 0.2) (layer "F.Cu") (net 7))
 (segment (start 162.401 102.199) (end 162.401 104.62611) (width 0.2) (layer "F.Cu") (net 7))
 (segment (start 161.65 104.2) (end 161.65 101.3) (width 0.2) (layer "F.Cu") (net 6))
 (segment (start 161.899999 96.4) (end 161.1625 96.4) (width 0.2) (layer "F.Cu") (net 6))
 (segment (start 160.124 95.277056) (end 160.601056 94.8) (width 0.2) (layer "F.Cu") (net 6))
 (segment (start 161.65 101.3) (end 163.95 99) (width 0.2) (layer "F.Cu") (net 6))
 (segment (start 160.601056 96.4) (end 160.124 95.922944) (width 0.2) (layer "F.Cu") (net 6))
 (segment (start 161.1625 96.4) (end 160.601056 96.4) (width 0.2) (layer "F.Cu") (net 6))
 (segment (start 164.575 107.6) (end 161.65 104.675) (width 0.2) (layer "F.Cu") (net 6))
 (segment (start 163.95 99) (end 163.95 98.450001) (width 0.2) (layer "F.Cu") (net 6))
 (segment (start 161.65 104.675) (end 161.65 104.2) (width 0.2) (layer "F.Cu") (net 6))
 (segment (start 167.05 107.6) (end 164.575 107.6) (width 0.2) (layer "F.Cu") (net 6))
 (segment (start 160.601056 94.8) (end 161.1625 94.8) (width 0.2) (layer "F.Cu") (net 6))
 (segment (start 157.2 104.2) (end 161.65 104.2) (width 0.2) (layer "F.Cu") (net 6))
 (segment (start 160.124 95.922944) (end 160.124 95.277056) (width 0.2) (layer "F.Cu") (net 6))
 (segment (start 163.95 98.450001) (end 161.899999 96.4) (width 0.2) (layer "F.Cu") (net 6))
 (segment (start 160.377056 91.024) (end 165.624 91.024) (width 0.2) (layer "F.Cu") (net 32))
 (segment (start 159.723 97.121944) (end 159.723 91.678056) (width 0.2) (layer "F.Cu") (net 32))
 (segment (start 160.377056 97.776) (end 159.723 97.121944) (width 0.2) (layer "F.Cu") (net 32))
 (segment (start 160.377056 99.346888) (end 160.377056 97.776) (width 0.2) (layer "F.Cu") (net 32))
 (segment (start 159.9849 108.201) (end 156.4615 104.6776) (width 0.2) (layer "F.Cu") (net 32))
 (segment (start 167.05 105.06) (end 168.024999 105.06) (width 0.2) (layer "F.Cu") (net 32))
 (segment (start 159.723 91.678056) (end 160.377056 91.024) (width 0.2) (layer "F.Cu") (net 32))
 (segment (start 156.4615 103.262444) (end 160.377056 99.346888) (width 0.2) (layer "F.Cu") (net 32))
 (segment (start 168.024999 105.06) (end 168.326 105.361001) (width 0.2) (layer "F.Cu") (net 32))
 (segment (start 165.624 91.024) (end 167.4 92.8) (width 0.2) (layer "F.Cu") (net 32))
 (segment (start 168.326 105.361001) (end 168.326 107.940968) (width 0.2) (layer "F.Cu") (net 32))
 (segment (start 165.2 92.8) (end 167.4 92.8) (width 0.2) (layer "F.Cu") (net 32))
 (segment (start 168.326 107.940968) (end 168.065968 108.201) (width 0.2) (layer "F.Cu") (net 32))
 (segment (start 168.065968 108.201) (end 159.9849 108.201) (width 0.2) (layer "F.Cu") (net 32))
 (segment (start 156.4615 104.6776) (end 156.4615 103.262444) (width 0.2) (layer "F.Cu") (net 32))
 (segment (start 171.735 92.8) (end 172 92.535) (width 0.2) (layer "F.Cu") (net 2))
 (segment (start 169.05 92.8) (end 171.735 92.8) (width 0.2) (layer "F.Cu") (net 2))
 (segment (start 173.276 106.670968) (end 172.346968 107.6) (width 0.2) (layer "F.Cu") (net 23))
 (segment (start 163.55 92.8) (end 164.349 93.599) (width 0.2) (layer "F.Cu") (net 23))
 (segment (start 163.15 92.4) (end 163.55 92.8) (width 0.2) (layer "F.Cu") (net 23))
 (segment (start 173.276 94.049) (end 173.276 106.670968) (width 0.2) (layer "F.Cu") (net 23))
 (segment (start 170.524 93.599) (end 170.849 93.924) (width 0.2) (layer "F.Cu") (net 23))
 (segment (start 170.849 93.924) (end 173.151 93.924) (width 0.2) (layer "F.Cu") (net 23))
 (segment (start 173.151 93.924) (end 173.276 94.049) (width 0.2) (layer "F.Cu") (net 23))
 (segment (start 161.1625 92.4) (end 163.15 92.4) (width 0.2) (layer "F.Cu") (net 23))
 (segment (start 164.349 93.599) (end 170.524 93.599) (width 0.2) (layer "F.Cu") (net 23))
 (segment (start 172.346968 107.6) (end 172 107.6) (width 0.2) (layer "F.Cu") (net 23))
 (segment (start 158.6 109.4) (end 160.6 109.4) (width 0.2) (layer "F.Cu") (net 5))
 (segment (start 153.876 93.677056) (end 153.876 94.498999) (width 0.2) (layer "F.Cu") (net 5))
 (segment (start 153.398944 93.2) (end 153.876 93.677056) (width 0.2) (layer "F.Cu") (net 5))
 (segment (start 150.465 94.8) (end 152.8375 94.8) (width 0.2) (layer "F.Cu") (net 5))
 (segment (start 148.4 96.865) (end 150.465 94.8) (width 0.2) (layer "F.Cu") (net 5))
 (segment (start 153.574999 94.8) (end 152.8375 94.8) (width 0.2) (layer "F.Cu") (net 5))
 (segment (start 158.6 109.4) (end 158.2 109.8) (width 0.2) (layer "F.Cu") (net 5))
 (segment (start 153.876 94.498999) (end 153.574999 94.8) (width 0.2) (layer "F.Cu") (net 5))
 (segment (start 152.8375 93.2) (end 153.398944 93.2) (width 0.2) (layer "F.Cu") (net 5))
 (via (at 160.6 109.4) (size 0.6) (drill 0.3) (layers "F.Cu" "B.Cu") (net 5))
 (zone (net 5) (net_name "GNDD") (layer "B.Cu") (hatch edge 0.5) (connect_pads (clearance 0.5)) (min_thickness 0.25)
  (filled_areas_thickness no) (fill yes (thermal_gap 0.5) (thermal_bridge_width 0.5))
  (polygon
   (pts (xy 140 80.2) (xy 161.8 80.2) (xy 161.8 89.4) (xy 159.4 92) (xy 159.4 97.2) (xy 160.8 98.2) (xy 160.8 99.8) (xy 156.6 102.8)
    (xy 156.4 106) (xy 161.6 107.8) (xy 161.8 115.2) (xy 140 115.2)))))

